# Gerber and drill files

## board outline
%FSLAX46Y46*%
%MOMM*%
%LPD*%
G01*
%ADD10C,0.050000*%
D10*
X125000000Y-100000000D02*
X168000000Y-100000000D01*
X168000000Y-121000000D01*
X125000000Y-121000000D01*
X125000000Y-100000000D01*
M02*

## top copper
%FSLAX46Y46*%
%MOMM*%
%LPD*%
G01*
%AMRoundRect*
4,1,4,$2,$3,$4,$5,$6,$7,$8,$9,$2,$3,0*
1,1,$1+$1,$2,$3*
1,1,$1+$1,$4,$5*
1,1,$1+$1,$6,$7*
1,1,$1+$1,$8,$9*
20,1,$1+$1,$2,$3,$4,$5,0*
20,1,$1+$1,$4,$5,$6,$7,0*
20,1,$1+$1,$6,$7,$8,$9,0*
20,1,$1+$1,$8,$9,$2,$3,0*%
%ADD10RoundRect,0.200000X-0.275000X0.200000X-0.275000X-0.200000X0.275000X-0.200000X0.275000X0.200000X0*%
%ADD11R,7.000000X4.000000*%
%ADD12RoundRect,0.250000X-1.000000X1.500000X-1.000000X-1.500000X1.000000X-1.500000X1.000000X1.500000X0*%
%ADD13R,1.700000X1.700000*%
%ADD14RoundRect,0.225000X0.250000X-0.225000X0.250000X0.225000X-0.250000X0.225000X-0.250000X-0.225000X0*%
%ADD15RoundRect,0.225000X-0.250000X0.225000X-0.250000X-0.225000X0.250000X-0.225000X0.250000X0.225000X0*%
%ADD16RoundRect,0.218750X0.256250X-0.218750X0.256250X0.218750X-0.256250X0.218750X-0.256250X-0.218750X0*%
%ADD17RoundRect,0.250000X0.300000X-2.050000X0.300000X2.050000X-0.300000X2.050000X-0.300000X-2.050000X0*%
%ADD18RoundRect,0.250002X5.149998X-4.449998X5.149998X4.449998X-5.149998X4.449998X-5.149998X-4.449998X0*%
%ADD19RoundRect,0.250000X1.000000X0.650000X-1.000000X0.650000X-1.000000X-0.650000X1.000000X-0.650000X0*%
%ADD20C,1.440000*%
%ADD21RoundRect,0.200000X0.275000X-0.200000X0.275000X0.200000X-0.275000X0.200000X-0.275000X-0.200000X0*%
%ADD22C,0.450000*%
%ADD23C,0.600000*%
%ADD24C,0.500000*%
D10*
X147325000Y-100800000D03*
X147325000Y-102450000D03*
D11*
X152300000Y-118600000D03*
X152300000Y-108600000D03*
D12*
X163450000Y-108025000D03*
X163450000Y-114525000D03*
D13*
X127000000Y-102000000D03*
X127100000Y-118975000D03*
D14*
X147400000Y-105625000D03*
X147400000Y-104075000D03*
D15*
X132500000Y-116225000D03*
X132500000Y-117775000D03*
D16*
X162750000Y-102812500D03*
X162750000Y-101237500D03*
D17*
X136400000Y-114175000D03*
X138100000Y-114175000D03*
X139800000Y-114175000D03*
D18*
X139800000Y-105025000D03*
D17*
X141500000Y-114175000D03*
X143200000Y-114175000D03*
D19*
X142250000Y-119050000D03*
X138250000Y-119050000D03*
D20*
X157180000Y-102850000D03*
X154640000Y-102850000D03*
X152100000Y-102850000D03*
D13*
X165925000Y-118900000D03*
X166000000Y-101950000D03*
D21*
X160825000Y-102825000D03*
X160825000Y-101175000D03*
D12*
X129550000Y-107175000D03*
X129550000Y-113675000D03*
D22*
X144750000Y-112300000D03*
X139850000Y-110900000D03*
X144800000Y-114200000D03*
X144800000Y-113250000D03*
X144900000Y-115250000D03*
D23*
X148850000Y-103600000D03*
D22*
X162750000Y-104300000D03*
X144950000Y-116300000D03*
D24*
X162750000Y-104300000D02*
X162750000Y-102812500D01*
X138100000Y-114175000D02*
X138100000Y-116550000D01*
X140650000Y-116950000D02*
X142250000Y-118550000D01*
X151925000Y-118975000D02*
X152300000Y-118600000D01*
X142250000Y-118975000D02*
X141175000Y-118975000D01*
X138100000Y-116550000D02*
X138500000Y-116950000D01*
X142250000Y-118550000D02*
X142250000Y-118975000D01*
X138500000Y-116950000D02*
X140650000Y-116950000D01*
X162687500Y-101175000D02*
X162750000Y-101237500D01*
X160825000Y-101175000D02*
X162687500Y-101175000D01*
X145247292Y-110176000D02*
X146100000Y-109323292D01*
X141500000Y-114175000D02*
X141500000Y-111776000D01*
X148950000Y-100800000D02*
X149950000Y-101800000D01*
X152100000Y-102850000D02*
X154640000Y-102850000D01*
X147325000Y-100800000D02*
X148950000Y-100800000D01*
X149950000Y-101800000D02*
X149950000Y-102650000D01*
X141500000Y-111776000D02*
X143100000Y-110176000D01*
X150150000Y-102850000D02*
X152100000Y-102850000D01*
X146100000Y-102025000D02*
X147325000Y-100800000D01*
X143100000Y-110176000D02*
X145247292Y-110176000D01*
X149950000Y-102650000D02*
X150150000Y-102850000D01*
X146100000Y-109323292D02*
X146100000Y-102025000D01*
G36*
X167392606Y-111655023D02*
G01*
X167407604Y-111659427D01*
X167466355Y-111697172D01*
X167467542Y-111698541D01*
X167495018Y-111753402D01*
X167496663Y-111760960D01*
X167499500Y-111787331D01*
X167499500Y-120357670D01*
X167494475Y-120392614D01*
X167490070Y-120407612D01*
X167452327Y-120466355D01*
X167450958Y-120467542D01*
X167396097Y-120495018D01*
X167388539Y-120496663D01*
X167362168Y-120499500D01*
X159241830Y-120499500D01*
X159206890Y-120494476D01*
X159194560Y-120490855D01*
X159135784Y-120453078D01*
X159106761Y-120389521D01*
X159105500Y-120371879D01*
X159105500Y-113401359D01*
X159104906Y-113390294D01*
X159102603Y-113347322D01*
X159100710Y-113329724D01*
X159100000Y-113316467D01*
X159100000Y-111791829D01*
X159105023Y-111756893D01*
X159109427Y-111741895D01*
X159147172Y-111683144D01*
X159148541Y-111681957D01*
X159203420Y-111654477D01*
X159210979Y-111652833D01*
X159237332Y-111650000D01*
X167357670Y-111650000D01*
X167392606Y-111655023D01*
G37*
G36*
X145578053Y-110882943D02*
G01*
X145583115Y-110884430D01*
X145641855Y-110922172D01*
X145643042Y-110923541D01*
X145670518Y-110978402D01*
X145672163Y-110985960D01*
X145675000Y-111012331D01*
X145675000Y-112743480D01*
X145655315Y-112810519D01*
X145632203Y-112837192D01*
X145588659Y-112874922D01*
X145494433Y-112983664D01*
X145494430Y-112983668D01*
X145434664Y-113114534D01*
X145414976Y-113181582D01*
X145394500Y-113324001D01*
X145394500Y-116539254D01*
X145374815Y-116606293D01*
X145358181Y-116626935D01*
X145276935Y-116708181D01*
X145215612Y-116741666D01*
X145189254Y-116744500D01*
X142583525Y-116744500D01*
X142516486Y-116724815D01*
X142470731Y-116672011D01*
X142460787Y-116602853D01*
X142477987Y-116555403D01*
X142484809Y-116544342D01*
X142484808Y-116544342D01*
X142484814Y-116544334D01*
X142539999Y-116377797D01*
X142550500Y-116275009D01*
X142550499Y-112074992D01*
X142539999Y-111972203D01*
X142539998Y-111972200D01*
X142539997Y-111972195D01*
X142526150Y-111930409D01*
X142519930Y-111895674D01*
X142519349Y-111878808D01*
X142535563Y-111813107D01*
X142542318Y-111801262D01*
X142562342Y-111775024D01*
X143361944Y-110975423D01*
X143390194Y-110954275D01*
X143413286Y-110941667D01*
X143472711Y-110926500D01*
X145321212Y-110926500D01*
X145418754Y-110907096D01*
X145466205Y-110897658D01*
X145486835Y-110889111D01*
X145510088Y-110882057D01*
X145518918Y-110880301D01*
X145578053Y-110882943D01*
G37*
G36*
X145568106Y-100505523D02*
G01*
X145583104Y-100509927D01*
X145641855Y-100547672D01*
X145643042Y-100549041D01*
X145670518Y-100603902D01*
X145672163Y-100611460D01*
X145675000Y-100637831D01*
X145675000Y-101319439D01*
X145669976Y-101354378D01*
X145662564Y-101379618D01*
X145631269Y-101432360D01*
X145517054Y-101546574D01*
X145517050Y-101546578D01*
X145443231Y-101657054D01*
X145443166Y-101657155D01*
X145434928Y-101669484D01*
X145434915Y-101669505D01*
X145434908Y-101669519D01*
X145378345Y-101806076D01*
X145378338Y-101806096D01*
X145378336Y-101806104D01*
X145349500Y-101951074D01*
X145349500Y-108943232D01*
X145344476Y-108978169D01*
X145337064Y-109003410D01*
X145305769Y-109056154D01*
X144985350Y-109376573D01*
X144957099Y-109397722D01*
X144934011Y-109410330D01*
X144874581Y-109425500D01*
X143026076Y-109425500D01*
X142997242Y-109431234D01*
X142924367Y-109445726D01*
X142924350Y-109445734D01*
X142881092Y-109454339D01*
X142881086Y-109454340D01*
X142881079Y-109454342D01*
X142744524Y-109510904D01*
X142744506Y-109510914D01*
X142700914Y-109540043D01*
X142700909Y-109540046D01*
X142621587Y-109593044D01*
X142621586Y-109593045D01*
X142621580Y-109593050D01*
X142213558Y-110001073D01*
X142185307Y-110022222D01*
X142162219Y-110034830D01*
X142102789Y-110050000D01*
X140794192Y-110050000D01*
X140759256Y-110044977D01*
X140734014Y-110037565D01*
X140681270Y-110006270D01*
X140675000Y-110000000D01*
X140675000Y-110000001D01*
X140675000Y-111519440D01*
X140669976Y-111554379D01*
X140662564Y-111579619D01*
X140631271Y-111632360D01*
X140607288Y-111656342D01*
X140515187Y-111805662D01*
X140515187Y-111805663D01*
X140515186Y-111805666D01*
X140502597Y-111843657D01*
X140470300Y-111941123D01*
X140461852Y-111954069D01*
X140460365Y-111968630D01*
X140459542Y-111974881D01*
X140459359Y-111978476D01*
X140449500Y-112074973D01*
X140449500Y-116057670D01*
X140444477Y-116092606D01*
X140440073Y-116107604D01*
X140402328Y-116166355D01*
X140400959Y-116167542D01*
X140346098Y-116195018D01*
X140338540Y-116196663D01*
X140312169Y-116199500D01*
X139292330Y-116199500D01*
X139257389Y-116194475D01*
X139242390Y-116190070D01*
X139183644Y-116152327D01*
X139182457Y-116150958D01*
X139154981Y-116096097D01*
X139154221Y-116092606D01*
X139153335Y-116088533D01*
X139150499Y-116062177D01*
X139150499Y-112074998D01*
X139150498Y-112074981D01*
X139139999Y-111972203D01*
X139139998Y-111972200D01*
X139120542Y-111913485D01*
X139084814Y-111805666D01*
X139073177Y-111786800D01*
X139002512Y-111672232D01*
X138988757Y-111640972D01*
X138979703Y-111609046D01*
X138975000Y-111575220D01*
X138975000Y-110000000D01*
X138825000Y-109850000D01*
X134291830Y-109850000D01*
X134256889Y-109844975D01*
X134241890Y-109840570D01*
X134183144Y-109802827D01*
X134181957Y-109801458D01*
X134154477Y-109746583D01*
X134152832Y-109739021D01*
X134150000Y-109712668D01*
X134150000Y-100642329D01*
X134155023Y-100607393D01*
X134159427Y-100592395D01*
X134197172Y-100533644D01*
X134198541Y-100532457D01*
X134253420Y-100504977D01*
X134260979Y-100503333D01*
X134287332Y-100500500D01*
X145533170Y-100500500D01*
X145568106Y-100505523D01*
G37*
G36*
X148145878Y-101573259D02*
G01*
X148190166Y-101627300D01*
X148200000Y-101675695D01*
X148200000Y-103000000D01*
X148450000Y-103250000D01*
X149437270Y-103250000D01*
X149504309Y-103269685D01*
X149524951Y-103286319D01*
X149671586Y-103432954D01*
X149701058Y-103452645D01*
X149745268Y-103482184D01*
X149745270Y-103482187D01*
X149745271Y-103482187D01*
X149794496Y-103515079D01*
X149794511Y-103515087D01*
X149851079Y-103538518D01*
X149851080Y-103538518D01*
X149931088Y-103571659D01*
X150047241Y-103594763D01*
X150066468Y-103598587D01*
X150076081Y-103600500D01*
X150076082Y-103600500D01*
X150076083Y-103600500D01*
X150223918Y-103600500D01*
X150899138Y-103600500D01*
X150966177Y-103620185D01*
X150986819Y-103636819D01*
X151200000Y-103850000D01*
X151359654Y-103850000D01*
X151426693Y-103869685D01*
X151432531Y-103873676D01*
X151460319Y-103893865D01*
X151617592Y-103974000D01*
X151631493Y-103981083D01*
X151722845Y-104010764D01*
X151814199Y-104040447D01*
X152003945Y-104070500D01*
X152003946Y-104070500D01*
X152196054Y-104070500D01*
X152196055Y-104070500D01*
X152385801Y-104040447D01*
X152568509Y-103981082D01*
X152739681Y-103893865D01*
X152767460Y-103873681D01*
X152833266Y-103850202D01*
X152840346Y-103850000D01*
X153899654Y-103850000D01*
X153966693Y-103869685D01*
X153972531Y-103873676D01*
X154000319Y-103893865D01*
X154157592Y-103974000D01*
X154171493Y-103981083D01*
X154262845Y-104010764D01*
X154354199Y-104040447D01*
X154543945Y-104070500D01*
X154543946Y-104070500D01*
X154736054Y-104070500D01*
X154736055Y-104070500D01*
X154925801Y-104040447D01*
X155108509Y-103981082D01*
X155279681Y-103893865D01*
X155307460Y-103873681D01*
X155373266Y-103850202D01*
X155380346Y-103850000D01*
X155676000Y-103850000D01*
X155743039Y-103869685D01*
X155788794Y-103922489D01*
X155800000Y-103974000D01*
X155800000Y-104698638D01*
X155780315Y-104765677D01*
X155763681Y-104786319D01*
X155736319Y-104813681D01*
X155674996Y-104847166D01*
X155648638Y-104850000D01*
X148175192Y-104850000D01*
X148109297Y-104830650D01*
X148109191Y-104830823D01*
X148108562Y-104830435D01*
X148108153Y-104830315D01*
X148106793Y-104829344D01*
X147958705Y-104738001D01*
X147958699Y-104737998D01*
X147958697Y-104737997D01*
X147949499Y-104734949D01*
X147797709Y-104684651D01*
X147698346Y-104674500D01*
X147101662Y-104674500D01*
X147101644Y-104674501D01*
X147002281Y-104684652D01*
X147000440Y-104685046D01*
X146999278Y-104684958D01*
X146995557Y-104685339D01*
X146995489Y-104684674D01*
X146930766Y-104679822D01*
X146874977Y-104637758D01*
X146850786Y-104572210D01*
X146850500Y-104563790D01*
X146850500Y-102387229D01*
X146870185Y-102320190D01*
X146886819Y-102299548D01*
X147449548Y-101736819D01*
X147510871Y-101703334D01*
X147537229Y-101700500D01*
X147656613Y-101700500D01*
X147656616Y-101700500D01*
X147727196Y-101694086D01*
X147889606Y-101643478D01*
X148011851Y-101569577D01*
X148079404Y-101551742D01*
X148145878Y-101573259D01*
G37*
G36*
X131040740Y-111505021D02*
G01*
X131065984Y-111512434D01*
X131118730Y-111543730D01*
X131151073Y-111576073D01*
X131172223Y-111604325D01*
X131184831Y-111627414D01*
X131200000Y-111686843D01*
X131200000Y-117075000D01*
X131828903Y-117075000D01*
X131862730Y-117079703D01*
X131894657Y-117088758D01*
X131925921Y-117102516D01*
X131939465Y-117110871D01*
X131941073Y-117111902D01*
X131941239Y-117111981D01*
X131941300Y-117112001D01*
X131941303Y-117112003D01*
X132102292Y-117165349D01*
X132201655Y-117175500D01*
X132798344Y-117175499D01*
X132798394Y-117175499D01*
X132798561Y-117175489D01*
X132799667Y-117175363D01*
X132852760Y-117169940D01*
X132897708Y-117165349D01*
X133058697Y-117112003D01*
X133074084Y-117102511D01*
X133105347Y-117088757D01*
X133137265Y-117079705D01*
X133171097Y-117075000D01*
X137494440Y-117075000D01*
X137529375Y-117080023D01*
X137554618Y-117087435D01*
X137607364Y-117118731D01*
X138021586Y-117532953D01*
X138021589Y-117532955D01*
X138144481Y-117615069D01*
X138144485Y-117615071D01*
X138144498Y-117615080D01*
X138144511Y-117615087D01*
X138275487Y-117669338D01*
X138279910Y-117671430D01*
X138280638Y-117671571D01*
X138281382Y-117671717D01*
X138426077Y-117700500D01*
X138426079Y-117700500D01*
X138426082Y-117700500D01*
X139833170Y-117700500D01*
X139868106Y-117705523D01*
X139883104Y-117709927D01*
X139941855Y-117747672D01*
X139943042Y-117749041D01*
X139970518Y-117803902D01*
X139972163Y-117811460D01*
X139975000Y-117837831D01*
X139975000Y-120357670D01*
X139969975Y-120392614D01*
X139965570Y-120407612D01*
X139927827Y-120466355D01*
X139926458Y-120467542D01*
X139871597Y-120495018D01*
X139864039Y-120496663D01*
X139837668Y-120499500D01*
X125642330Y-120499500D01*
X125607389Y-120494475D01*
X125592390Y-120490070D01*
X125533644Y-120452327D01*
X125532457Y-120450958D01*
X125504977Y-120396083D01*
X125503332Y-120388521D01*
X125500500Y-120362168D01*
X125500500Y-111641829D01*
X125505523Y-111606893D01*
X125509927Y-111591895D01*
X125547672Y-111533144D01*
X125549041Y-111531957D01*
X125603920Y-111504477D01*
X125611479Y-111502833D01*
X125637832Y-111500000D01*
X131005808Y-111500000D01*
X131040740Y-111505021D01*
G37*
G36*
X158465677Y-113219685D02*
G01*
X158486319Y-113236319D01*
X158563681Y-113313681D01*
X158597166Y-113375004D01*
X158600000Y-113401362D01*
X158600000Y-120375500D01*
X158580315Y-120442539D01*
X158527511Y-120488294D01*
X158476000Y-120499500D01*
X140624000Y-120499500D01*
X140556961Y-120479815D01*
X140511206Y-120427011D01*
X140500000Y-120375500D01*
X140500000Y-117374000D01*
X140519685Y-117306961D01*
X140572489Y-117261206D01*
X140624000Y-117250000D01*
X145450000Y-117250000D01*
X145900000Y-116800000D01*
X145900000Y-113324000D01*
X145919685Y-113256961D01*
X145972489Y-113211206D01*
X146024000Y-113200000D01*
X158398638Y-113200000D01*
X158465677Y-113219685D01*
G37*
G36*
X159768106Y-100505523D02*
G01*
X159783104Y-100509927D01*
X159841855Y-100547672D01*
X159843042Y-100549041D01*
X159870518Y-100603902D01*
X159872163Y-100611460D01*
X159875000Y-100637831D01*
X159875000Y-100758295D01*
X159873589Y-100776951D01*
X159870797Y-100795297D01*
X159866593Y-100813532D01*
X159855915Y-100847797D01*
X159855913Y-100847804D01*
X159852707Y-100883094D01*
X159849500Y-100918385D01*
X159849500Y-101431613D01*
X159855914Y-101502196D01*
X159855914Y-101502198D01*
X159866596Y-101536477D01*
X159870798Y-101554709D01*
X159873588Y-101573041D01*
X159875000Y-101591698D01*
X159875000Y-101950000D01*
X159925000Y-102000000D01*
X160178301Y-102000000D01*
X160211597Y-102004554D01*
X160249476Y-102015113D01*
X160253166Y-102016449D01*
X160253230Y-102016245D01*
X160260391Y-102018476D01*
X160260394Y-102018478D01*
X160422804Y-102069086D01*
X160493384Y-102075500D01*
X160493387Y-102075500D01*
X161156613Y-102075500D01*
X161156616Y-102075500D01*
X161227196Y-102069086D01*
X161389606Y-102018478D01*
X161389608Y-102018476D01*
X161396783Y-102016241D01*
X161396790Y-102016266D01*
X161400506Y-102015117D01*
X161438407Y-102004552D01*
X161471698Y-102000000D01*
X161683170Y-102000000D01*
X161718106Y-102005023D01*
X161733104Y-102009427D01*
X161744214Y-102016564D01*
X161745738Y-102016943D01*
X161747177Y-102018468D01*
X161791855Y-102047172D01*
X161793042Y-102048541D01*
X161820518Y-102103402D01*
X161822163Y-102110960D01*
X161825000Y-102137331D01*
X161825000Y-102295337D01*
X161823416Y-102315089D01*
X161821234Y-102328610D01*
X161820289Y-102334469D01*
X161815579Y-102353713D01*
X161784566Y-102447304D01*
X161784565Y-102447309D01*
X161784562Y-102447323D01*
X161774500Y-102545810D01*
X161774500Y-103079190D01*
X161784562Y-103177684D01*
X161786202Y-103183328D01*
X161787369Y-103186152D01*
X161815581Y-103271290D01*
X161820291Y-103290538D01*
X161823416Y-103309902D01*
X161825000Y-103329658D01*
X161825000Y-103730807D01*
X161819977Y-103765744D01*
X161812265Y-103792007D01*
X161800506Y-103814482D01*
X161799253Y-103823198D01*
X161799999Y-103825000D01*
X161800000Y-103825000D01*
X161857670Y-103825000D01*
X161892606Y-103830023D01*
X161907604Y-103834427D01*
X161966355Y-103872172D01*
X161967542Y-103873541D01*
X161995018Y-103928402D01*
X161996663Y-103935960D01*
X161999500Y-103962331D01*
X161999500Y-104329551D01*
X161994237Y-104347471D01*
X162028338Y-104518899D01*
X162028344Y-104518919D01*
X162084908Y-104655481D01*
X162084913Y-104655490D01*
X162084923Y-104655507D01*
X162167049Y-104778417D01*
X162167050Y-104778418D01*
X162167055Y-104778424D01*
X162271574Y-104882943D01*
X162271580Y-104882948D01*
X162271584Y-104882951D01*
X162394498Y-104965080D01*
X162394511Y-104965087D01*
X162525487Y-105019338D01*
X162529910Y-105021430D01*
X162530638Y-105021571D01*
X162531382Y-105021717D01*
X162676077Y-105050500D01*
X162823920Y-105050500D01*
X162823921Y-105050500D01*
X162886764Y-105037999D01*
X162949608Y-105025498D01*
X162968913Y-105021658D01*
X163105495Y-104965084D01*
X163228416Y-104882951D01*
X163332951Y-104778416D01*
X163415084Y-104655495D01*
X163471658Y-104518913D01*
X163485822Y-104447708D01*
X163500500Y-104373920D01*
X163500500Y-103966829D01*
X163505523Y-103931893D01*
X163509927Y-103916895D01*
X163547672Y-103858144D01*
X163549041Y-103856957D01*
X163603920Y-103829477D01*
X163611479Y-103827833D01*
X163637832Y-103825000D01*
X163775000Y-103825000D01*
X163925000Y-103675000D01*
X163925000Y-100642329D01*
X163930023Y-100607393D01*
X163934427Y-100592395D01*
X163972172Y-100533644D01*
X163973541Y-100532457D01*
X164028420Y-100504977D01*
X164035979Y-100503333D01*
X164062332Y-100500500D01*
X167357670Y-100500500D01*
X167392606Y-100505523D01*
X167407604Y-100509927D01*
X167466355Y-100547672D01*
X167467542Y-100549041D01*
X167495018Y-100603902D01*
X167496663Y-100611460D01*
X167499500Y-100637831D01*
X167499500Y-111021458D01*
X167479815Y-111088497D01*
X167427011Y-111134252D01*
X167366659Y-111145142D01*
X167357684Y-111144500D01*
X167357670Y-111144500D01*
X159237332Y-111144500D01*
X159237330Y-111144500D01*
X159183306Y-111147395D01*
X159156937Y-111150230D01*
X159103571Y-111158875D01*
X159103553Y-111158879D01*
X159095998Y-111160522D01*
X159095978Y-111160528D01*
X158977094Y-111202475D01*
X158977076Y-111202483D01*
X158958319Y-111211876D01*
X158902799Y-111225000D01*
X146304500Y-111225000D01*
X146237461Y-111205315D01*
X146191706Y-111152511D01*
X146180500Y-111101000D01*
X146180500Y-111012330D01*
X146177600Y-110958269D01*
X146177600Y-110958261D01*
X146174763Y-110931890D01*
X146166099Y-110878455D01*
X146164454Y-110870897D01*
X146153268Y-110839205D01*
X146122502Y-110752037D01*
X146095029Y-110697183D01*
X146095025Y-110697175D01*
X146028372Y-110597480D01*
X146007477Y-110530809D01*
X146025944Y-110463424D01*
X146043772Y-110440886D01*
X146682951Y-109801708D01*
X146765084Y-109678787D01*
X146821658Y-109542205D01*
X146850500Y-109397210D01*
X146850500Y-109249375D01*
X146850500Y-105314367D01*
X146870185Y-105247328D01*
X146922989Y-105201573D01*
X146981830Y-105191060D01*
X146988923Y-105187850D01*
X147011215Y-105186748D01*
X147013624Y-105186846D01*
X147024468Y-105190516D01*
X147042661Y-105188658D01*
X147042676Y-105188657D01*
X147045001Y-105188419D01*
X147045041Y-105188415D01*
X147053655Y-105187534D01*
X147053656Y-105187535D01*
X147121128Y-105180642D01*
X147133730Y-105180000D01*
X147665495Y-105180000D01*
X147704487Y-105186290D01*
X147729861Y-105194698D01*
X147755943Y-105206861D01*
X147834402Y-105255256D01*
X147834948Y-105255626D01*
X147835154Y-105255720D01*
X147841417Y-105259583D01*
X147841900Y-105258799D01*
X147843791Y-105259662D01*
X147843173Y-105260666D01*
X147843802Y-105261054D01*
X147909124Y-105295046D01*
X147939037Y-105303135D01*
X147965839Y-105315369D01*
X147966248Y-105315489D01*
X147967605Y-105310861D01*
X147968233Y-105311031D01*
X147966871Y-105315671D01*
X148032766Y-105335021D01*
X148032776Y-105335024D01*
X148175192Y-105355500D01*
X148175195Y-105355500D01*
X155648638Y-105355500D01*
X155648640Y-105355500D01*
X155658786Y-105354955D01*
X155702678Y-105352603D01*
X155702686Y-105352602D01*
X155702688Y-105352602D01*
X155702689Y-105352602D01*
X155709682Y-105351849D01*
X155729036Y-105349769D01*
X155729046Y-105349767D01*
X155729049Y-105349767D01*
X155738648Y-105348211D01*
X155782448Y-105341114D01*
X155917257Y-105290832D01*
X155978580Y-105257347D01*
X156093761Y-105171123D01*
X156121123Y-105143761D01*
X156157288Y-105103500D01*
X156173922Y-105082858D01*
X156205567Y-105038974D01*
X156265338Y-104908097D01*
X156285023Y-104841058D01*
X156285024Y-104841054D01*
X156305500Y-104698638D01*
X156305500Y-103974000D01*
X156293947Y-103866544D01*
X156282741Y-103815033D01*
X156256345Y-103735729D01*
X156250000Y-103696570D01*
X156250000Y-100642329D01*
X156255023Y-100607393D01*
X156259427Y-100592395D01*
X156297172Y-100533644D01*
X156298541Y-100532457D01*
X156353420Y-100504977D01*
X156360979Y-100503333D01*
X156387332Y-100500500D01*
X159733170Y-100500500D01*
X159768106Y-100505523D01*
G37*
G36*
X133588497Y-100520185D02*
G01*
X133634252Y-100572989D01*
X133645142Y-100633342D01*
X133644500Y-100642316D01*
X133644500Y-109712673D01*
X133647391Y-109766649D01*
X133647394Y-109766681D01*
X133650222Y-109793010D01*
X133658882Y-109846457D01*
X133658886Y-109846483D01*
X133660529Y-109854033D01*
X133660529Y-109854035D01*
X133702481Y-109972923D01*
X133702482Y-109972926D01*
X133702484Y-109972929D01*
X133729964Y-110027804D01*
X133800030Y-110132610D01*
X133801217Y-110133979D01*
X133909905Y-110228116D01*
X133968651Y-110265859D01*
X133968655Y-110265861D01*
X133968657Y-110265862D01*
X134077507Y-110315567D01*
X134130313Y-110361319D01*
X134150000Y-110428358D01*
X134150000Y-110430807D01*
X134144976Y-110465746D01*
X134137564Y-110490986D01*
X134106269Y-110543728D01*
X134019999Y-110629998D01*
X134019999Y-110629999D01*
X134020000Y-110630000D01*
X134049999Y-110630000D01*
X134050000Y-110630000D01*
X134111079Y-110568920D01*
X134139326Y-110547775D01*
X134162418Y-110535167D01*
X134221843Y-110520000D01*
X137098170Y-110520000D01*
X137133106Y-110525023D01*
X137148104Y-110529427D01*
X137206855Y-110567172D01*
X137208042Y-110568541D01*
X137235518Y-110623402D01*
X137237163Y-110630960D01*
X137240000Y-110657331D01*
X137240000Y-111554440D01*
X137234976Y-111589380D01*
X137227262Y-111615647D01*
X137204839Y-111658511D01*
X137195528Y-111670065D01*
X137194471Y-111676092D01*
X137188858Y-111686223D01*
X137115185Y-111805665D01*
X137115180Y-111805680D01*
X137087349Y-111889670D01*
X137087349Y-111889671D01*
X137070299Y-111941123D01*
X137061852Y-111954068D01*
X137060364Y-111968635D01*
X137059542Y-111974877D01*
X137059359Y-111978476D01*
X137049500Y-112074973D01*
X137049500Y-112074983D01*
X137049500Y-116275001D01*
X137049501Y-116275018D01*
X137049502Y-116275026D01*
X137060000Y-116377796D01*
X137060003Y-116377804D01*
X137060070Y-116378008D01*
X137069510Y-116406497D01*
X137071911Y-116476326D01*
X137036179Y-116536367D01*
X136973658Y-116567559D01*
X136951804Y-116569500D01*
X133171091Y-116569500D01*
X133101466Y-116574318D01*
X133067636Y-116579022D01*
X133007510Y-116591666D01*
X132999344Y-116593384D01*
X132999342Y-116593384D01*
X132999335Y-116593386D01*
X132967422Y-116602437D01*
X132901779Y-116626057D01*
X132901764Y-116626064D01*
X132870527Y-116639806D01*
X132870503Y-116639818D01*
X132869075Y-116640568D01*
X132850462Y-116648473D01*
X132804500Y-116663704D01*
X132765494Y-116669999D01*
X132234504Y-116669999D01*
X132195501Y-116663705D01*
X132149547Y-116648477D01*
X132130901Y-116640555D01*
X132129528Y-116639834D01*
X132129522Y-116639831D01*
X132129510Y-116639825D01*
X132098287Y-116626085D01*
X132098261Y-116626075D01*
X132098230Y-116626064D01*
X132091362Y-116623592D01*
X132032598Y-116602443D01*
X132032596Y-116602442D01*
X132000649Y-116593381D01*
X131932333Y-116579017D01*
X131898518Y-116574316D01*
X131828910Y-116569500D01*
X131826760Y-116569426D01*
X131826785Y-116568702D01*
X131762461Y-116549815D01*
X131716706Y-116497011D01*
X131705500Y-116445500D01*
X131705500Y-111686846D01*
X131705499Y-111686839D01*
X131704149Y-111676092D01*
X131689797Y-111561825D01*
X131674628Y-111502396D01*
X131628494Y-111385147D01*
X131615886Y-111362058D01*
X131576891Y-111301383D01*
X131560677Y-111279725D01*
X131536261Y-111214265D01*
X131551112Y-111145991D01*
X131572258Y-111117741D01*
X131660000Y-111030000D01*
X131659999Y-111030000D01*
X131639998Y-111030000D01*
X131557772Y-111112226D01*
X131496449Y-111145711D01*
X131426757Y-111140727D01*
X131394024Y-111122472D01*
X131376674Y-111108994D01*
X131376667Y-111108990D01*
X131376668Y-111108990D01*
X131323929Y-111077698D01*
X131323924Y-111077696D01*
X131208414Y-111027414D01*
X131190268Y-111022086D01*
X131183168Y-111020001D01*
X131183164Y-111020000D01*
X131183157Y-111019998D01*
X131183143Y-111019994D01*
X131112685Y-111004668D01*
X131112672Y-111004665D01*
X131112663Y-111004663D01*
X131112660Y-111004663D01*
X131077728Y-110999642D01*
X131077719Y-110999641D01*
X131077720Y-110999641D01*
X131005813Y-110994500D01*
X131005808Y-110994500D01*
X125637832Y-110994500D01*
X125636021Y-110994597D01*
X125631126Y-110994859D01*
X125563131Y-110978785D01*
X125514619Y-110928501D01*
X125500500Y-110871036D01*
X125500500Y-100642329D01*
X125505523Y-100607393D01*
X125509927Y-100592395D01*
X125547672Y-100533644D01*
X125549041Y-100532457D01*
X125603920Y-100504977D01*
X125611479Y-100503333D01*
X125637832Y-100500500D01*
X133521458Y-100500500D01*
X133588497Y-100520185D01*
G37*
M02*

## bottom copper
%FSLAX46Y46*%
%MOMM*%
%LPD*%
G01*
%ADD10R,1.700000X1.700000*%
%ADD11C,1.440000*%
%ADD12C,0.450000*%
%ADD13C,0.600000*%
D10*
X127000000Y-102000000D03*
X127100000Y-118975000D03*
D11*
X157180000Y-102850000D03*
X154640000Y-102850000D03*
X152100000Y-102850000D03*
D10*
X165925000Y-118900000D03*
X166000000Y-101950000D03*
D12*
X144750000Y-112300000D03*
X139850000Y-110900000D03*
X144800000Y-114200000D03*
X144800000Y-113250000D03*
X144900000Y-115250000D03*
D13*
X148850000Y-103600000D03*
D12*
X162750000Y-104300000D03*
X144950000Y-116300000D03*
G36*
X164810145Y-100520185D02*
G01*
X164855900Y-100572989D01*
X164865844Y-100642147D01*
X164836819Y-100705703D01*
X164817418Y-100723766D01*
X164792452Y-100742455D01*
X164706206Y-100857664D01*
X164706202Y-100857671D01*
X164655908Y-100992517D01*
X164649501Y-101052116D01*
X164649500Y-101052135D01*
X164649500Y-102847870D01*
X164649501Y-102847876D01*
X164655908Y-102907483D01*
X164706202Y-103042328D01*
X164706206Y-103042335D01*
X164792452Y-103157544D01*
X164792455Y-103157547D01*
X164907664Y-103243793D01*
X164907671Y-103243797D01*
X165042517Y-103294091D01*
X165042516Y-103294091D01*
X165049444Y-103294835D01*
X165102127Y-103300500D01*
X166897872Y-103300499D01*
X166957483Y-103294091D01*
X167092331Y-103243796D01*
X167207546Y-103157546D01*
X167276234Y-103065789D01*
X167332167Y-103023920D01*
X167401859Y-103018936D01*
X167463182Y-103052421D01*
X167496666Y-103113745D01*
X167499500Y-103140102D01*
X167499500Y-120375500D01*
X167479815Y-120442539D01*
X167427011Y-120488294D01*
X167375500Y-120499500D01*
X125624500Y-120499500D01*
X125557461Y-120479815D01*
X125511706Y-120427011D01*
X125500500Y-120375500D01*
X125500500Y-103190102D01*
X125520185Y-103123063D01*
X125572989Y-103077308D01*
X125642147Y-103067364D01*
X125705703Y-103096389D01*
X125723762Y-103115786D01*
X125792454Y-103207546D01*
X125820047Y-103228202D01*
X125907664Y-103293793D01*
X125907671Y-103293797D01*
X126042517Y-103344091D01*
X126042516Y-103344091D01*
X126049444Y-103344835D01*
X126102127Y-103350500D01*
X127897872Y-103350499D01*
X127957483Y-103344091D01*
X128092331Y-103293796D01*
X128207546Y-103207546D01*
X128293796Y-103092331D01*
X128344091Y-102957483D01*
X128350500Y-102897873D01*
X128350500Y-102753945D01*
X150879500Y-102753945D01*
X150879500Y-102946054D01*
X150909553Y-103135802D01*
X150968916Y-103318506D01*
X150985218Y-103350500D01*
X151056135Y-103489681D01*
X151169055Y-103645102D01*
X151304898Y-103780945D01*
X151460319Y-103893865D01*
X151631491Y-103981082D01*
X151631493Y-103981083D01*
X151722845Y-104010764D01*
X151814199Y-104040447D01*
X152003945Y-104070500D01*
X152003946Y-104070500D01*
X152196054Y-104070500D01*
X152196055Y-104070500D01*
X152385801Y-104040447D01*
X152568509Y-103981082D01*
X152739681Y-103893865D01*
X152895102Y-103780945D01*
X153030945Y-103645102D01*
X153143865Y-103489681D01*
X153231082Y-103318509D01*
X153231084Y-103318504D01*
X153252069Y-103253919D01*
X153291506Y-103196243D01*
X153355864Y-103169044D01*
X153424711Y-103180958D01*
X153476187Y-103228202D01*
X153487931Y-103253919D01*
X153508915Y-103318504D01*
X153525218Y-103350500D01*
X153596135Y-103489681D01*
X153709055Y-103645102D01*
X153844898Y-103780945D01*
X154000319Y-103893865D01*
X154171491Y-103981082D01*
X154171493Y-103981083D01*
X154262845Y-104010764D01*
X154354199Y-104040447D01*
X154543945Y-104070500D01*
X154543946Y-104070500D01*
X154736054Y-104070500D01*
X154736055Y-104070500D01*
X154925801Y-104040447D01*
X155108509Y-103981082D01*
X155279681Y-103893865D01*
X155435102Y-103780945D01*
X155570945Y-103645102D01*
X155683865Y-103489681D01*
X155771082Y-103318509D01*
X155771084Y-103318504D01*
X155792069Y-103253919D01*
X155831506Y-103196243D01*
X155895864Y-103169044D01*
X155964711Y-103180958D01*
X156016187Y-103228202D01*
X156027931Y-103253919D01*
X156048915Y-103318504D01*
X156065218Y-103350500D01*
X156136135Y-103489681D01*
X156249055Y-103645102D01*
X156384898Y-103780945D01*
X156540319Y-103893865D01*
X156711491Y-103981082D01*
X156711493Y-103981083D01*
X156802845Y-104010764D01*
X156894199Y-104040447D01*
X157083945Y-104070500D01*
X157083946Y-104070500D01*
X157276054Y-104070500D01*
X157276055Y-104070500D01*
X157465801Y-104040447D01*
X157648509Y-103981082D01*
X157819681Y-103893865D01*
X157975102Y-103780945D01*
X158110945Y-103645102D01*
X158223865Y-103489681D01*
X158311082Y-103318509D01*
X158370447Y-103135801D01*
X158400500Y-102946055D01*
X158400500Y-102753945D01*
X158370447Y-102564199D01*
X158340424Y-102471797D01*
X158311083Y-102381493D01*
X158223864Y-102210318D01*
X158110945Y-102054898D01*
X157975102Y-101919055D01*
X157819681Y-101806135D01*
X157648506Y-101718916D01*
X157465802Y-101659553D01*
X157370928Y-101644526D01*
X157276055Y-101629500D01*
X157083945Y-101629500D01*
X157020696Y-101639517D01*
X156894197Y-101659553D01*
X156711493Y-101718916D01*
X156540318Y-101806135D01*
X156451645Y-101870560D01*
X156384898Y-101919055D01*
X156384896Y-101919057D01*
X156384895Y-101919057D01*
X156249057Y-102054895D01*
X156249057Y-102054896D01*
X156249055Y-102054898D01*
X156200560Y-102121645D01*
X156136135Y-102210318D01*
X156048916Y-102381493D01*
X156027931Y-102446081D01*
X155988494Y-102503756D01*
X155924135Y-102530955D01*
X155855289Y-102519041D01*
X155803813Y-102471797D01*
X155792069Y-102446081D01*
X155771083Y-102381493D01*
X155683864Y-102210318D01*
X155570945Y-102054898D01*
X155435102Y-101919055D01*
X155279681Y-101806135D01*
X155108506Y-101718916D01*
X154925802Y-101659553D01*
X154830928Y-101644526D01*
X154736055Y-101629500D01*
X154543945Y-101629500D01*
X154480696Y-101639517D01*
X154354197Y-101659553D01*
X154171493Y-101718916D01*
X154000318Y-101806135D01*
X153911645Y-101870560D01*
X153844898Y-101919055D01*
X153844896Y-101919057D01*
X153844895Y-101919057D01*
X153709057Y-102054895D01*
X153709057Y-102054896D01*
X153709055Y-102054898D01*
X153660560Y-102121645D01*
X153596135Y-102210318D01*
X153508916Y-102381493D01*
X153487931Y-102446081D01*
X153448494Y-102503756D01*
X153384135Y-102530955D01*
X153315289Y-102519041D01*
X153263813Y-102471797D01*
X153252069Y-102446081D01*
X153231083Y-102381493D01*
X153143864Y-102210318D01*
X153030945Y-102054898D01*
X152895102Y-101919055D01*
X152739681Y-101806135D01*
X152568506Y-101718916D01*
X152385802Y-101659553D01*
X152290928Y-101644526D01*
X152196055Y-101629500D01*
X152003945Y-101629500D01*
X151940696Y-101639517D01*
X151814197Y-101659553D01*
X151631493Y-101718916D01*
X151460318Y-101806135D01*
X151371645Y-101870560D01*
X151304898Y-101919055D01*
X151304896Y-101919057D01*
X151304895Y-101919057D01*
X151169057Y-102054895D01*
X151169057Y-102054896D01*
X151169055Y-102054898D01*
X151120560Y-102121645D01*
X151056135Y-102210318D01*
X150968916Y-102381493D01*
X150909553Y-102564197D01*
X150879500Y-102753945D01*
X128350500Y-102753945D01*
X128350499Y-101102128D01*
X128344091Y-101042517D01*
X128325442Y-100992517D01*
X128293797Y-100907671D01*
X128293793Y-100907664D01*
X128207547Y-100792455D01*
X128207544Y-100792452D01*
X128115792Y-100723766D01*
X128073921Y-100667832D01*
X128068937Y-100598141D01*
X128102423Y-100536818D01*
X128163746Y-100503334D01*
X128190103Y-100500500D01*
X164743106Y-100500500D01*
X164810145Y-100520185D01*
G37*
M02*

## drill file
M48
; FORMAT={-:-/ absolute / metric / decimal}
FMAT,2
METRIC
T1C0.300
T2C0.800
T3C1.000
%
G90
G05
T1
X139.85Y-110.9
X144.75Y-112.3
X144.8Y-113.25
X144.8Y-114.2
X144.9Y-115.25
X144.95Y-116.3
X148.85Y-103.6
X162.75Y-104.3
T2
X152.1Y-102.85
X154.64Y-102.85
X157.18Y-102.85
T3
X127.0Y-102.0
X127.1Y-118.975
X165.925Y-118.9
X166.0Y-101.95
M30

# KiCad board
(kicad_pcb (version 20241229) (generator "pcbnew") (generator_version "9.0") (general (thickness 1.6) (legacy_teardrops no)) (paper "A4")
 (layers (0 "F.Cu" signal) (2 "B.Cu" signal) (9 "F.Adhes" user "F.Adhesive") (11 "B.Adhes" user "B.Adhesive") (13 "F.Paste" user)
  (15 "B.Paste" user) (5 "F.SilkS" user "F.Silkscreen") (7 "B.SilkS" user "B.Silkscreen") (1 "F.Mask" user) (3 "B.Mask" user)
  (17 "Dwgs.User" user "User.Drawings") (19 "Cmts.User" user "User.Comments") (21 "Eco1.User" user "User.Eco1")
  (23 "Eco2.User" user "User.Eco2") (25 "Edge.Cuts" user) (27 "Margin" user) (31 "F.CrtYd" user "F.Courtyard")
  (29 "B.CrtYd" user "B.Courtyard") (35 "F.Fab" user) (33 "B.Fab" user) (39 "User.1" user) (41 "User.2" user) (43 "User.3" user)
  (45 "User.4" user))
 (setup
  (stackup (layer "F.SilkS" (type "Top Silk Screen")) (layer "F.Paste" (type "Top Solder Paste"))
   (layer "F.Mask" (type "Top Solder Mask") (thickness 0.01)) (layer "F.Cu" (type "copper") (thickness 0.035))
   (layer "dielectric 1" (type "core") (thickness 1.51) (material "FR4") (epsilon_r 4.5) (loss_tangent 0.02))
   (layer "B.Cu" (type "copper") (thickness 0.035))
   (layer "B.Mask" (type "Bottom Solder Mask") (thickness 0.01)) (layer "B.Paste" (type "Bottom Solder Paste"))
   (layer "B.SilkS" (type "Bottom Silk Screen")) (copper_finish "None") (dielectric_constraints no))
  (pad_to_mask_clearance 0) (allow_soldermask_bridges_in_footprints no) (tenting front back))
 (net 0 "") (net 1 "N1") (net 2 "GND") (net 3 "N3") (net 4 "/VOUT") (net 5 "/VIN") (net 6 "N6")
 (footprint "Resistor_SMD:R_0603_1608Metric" (layer "F.Cu") (at 147.325 101.625 -90)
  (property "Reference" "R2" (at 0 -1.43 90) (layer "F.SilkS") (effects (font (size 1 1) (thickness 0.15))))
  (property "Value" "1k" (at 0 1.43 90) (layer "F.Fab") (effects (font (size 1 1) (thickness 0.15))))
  (pad "1" smd roundrect (at -0.825 0 270) (size 0.8 0.95) (layers "F.Cu" "F.Mask" "F.Paste") (roundrect_rratio 0.25) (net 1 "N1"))
  (pad "2" smd roundrect (at 0.825 0 270) (size 0.8 0.95) (layers "F.Cu" "F.Mask" "F.Paste") (roundrect_rratio 0.25) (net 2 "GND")))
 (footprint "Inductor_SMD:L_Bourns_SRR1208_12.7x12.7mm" (layer "F.Cu") (at 152.3 113.6 90)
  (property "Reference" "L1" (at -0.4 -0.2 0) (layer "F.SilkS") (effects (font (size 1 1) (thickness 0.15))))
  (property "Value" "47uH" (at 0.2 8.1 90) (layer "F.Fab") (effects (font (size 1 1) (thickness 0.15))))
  (pad "1" smd rect (at -5 0 90) (size 4 7) (layers "F.Cu" "F.Mask" "F.Paste") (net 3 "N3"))
  (pad "2" smd rect (at 5 0 90) (size 4 7) (layers "F.Cu" "F.Mask" "F.Paste") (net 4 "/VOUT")))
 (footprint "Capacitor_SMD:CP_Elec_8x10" (layer "F.Cu") (at 163.45 111.275 -90)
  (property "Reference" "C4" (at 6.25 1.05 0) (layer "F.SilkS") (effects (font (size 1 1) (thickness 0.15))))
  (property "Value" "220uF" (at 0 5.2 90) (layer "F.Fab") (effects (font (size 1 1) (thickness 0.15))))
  (pad "1" smd roundrect (at -3.25 0 270) (size 3.5 2.5) (layers "F.Cu" "F.Mask" "F.Paste") (roundrect_rratio 0.1) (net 4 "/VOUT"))
  (pad "2" smd roundrect (at 3.25 0 270) (size 3.5 2.5) (layers "F.Cu" "F.Mask" "F.Paste") (roundrect_rratio 0.1) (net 2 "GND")))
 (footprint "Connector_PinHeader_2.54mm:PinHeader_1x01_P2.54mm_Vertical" (layer "F.Cu") (at 127 102)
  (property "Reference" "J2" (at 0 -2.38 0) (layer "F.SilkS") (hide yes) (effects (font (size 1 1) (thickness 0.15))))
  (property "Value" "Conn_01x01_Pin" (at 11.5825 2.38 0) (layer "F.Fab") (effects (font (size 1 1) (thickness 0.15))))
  (pad "1" thru_hole rect (at 0 0) (size 1.7 1.7) (drill 1) (layers "*.Cu" "*.Mask") (remove_unused_layers no) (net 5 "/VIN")))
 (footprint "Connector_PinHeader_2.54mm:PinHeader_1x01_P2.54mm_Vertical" (layer "F.Cu") (at 127.1 118.975)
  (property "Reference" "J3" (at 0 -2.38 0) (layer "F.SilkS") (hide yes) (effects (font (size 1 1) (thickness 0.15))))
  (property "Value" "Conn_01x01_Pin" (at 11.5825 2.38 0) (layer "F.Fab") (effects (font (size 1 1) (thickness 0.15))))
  (pad "1" thru_hole rect (at 0 0) (size 1.7 1.7) (drill 1) (layers "*.Cu" "*.Mask") (remove_unused_layers no) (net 2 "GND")))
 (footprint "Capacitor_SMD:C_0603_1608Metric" (layer "F.Cu") (at 147.4 104.85 90)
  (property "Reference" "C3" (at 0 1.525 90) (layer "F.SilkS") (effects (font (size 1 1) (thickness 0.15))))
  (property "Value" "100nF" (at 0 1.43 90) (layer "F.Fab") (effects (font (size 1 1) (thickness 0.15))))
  (pad "1" smd roundrect (at -0.775 0 90) (size 0.9 0.95) (layers "F.Cu" "F.Mask" "F.Paste") (roundrect_rratio 0.25) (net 4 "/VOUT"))
  (pad "2" smd roundrect (at 0.775 0 90) (size 0.9 0.95) (layers "F.Cu" "F.Mask" "F.Paste") (roundrect_rratio 0.25) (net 2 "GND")))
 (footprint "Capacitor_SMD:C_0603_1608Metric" (layer "F.Cu") (at 132.5 117 -90)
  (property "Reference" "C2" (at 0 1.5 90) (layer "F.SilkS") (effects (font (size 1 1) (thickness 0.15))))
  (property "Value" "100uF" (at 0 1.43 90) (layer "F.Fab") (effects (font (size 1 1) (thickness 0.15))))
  (pad "1" smd roundrect (at -0.775 0 270) (size 0.9 0.95) (layers "F.Cu" "F.Mask" "F.Paste") (roundrect_rratio 0.25) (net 5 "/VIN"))
  (pad "2" smd roundrect (at 0.775 0 270) (size 0.9 0.95) (layers "F.Cu" "F.Mask" "F.Paste") (roundrect_rratio 0.25) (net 2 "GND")))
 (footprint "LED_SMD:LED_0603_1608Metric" (layer "F.Cu") (at 162.75 102.025 90)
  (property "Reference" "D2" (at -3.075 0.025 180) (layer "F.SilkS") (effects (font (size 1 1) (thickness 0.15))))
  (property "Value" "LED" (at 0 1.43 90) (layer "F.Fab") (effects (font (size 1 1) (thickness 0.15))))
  (pad "1" smd roundrect (at -0.7875 0 90) (size 0.875 0.95) (layers "F.Cu" "F.Mask" "F.Paste") (roundrect_rratio 0.25) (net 2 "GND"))
  (pad "2" smd roundrect (at 0.7875 0 90) (size 0.875 0.95) (layers "F.Cu" "F.Mask" "F.Paste") (roundrect_rratio 0.25) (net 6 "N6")))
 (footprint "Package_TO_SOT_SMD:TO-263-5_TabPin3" (layer "F.Cu") (at 139.8 106.525 90)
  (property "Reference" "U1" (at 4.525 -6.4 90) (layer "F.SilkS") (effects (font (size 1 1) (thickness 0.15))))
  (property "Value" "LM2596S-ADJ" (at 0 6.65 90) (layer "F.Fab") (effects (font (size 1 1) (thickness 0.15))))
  (pad "" smd roundrect (at -0.925 -2.775 90) (size 4.55 5.25) (layers "F.Paste") (roundrect_rratio 0.054945))
  (pad "" smd roundrect (at -0.925 2.775 90) (size 4.55 5.25) (layers "F.Paste") (roundrect_rratio 0.054945))
  (pad "" smd roundrect (at 3.925 -2.775 90) (size 4.55 5.25) (layers "F.Paste") (roundrect_rratio 0.054945))
  (pad "" smd roundrect (at 3.925 2.775 90) (size 4.55 5.25) (layers "F.Paste") (roundrect_rratio 0.054945))
  (pad "1" smd roundrect (at -7.65 -3.4 90) (size 4.6 1.1) (layers "F.Cu" "F.Mask" "F.Paste") (roundrect_rratio 0.227273) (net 5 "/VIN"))
  (pad "2" smd roundrect (at -7.65 -1.7 90) (size 4.6 1.1) (layers "F.Cu" "F.Mask" "F.Paste") (roundrect_rratio 0.227273) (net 3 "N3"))
  (pad "3" smd roundrect (at -7.65 0 90) (size 4.6 1.1) (layers "F.Cu" "F.Mask" "F.Paste") (roundrect_rratio 0.227273) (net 2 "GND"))
  (pad "3" smd roundrect (at 1.5 0 90) (size 9.4 10.8) (layers "F.Cu" "F.Mask") (roundrect_rratio 0.026596) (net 2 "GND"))
  (pad "4" smd roundrect (at -7.65 1.7 90) (size 4.6 1.1) (layers "F.Cu" "F.Mask" "F.Paste") (roundrect_rratio 0.227273) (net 1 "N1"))
  (pad "5" smd roundrect (at -7.65 3.4 90) (size 4.6 1.1) (layers "F.Cu" "F.Mask" "F.Paste") (roundrect_rratio 0.227273) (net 2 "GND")))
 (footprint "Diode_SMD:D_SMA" (layer "F.Cu") (at 140.25 119.05 180)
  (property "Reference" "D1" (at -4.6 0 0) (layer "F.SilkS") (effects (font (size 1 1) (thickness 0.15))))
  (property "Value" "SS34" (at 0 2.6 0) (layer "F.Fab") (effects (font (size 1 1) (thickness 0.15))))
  (pad "1" smd roundrect (at -2 0 180) (size 2.5 1.8) (layers "F.Cu" "F.Mask" "F.Paste") (roundrect_rratio 0.1388888889) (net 3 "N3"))
  (pad "2" smd roundrect (at 2 0 180) (size 2.5 1.8) (layers "F.Cu" "F.Mask" "F.Paste") (roundrect_rratio 0.1388888889) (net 2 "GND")))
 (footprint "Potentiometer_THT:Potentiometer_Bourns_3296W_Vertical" (layer "F.Cu") (at 157.18 102.85)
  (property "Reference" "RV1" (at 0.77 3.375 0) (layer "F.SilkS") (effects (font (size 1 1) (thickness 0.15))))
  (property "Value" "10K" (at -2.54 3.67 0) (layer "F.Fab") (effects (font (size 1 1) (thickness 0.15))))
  (pad "1" thru_hole circle (at 0 0) (size 1.44 1.44) (drill 0.8) (layers "*.Cu" "*.Mask") (remove_unused_layers no) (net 4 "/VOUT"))
  (pad "2" thru_hole circle (at -2.54 0) (size 1.44 1.44) (drill 0.8) (layers "*.Cu" "*.Mask") (remove_unused_layers no) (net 1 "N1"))
  (pad "3" thru_hole circle (at -5.08 0) (size 1.44 1.44) (drill 0.8) (layers "*.Cu" "*.Mask") (remove_unused_layers no) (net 1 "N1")))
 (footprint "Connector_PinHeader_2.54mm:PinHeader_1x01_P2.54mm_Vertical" (layer "F.Cu") (at 165.925 118.9)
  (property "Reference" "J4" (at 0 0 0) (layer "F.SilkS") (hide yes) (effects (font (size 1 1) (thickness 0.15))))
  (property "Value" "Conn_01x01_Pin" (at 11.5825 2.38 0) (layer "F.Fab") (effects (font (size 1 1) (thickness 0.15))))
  (pad "1" thru_hole rect (at 0 0) (size 1.7 1.7) (drill 1) (layers "*.Cu" "*.Mask") (remove_unused_layers no) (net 2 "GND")))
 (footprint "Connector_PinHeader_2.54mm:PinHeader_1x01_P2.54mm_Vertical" (layer "F.Cu") (at 166 101.95)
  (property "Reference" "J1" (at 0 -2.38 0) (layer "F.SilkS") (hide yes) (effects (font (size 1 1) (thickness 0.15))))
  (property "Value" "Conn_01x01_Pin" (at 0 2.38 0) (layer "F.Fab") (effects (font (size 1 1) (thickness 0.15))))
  (pad "1" thru_hole rect (at 0 0) (size 1.7 1.7) (drill 1) (layers "*.Cu" "*.Mask") (remove_unused_layers no) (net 4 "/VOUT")))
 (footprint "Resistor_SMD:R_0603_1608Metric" (layer "F.Cu") (at 160.825 102 90)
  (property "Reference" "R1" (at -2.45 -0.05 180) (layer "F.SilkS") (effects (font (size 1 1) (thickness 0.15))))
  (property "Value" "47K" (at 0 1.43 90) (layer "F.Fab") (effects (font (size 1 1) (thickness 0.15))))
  (pad "1" smd roundrect (at -0.825 0 90) (size 0.8 0.95) (layers "F.Cu" "F.Mask" "F.Paste") (roundrect_rratio 0.25) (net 4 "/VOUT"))
  (pad "2" smd roundrect (at 0.825 0 90) (size 0.8 0.95) (layers "F.Cu" "F.Mask" "F.Paste") (roundrect_rratio 0.25) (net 6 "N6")))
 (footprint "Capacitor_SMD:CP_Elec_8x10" (layer "F.Cu") (at 129.55 110.425 -90)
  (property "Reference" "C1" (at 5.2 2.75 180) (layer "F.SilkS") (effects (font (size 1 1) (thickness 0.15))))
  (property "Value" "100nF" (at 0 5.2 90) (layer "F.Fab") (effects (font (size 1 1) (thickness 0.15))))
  (pad "1" smd roundrect (at -3.25 0 270) (size 3.5 2.5) (layers "F.Cu" "F.Mask" "F.Paste") (roundrect_rratio 0.1) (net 5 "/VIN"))
  (pad "2" smd roundrect (at 3.25 0 270) (size 3.5 2.5) (layers "F.Cu" "F.Mask" "F.Paste") (roundrect_rratio 0.1) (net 2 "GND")))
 (gr_rect (start 125 100) (end 168 121) (stroke (width 0.05) (type default)) (fill no) (layer "Edge.Cuts"))
 (segment (start 162.75 104.3) (end 162.75 102.8125) (width 0.5) (layer "F.Cu") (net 2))
 (via (at 144.75 112.3) (size 0.45) (drill 0.3) (layers "F.Cu" "B.Cu") (free yes) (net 2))
 (via (at 139.85 110.9) (size 0.45) (drill 0.3) (layers "F.Cu" "B.Cu") (free yes) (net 2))
 (via (at 144.8 114.2) (size 0.45) (drill 0.3) (layers "F.Cu" "B.Cu") (free yes) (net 2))
 (via (at 144.8 113.25) (size 0.45) (drill 0.3) (layers "F.Cu" "B.Cu") (free yes) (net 2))
 (via (at 144.9 115.25) (size 0.45) (drill 0.3) (layers "F.Cu" "B.Cu") (free yes) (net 2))
 (via (at 148.85 103.6) (size 0.6) (drill 0.3) (layers "F.Cu" "B.Cu") (free yes) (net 2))
 (via (at 162.75 104.3) (size 0.45) (drill 0.3) (layers "F.Cu" "B.Cu") (free yes) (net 2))
 (via (at 144.95 116.3) (size 0.45) (drill 0.3) (layers "F.Cu" "B.Cu") (free yes) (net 2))
 (segment (start 138.1 114.175) (end 138.1 116.55) (width 0.5) (layer "F.Cu") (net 3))
 (segment (start 140.65 116.95) (end 142.25 118.55) (width 0.5) (layer "F.Cu") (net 3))
 (segment (start 151.925 118.975) (end 152.3 118.6) (width 0.5) (layer "F.Cu") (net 3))
 (segment (start 142.25 118.975) (end 141.175 118.975) (width 0.5) (layer "F.Cu") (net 3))
 (segment (start 138.1 116.55) (end 138.5 116.95) (width 0.5) (layer "F.Cu") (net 3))
 (segment (start 142.25 118.55) (end 142.25 118.975) (width 0.5) (layer "F.Cu") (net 3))
 (segment (start 138.5 116.95) (end 140.65 116.95) (width 0.5) (layer "F.Cu") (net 3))
 (segment (start 162.6875 101.175) (end 162.75 101.2375) (width 0.5) (layer "F.Cu") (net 6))
 (segment (start 160.825 101.175) (end 162.6875 101.175) (width 0.5) (layer "F.Cu") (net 6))
 (segment (start 145.247292 110.176) (end 146.1 109.323292) (width 0.5) (layer "F.Cu") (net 1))
 (segment (start 141.5 114.175) (end 141.5 111.776) (width 0.5) (layer "F.Cu") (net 1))
 (segment (start 148.95 100.8) (end 149.95 101.8) (width 0.5) (layer "F.Cu") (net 1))
 (segment (start 152.1 102.85) (end 154.64 102.85) (width 0.5) (layer "F.Cu") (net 1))
 (segment (start 147.325 100.8) (end 148.95 100.8) (width 0.5) (layer "F.Cu") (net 1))
 (segment (start 149.95 101.8) (end 149.95 102.65) (width 0.5) (layer "F.Cu") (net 1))
 (segment (start 141.5 111.776) (end 143.1 110.176) (width 0.5) (layer "F.Cu") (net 1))
 (segment (start 150.15 102.85) (end 152.1 102.85) (width 0.5) (layer "F.Cu") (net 1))
 (segment (start 146.1 102.025) (end 147.325 100.8) (width 0.5) (layer "F.Cu") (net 1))
 (segment (start 143.1 110.176) (end 145.247292 110.176) (width 0.5) (layer "F.Cu") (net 1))
 (segment (start 149.95 102.65) (end 150.15 102.85) (width 0.5) (layer "F.Cu") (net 1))
 (segment (start 146.1 109.323292) (end 146.1 102.025) (width 0.5) (layer "F.Cu") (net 1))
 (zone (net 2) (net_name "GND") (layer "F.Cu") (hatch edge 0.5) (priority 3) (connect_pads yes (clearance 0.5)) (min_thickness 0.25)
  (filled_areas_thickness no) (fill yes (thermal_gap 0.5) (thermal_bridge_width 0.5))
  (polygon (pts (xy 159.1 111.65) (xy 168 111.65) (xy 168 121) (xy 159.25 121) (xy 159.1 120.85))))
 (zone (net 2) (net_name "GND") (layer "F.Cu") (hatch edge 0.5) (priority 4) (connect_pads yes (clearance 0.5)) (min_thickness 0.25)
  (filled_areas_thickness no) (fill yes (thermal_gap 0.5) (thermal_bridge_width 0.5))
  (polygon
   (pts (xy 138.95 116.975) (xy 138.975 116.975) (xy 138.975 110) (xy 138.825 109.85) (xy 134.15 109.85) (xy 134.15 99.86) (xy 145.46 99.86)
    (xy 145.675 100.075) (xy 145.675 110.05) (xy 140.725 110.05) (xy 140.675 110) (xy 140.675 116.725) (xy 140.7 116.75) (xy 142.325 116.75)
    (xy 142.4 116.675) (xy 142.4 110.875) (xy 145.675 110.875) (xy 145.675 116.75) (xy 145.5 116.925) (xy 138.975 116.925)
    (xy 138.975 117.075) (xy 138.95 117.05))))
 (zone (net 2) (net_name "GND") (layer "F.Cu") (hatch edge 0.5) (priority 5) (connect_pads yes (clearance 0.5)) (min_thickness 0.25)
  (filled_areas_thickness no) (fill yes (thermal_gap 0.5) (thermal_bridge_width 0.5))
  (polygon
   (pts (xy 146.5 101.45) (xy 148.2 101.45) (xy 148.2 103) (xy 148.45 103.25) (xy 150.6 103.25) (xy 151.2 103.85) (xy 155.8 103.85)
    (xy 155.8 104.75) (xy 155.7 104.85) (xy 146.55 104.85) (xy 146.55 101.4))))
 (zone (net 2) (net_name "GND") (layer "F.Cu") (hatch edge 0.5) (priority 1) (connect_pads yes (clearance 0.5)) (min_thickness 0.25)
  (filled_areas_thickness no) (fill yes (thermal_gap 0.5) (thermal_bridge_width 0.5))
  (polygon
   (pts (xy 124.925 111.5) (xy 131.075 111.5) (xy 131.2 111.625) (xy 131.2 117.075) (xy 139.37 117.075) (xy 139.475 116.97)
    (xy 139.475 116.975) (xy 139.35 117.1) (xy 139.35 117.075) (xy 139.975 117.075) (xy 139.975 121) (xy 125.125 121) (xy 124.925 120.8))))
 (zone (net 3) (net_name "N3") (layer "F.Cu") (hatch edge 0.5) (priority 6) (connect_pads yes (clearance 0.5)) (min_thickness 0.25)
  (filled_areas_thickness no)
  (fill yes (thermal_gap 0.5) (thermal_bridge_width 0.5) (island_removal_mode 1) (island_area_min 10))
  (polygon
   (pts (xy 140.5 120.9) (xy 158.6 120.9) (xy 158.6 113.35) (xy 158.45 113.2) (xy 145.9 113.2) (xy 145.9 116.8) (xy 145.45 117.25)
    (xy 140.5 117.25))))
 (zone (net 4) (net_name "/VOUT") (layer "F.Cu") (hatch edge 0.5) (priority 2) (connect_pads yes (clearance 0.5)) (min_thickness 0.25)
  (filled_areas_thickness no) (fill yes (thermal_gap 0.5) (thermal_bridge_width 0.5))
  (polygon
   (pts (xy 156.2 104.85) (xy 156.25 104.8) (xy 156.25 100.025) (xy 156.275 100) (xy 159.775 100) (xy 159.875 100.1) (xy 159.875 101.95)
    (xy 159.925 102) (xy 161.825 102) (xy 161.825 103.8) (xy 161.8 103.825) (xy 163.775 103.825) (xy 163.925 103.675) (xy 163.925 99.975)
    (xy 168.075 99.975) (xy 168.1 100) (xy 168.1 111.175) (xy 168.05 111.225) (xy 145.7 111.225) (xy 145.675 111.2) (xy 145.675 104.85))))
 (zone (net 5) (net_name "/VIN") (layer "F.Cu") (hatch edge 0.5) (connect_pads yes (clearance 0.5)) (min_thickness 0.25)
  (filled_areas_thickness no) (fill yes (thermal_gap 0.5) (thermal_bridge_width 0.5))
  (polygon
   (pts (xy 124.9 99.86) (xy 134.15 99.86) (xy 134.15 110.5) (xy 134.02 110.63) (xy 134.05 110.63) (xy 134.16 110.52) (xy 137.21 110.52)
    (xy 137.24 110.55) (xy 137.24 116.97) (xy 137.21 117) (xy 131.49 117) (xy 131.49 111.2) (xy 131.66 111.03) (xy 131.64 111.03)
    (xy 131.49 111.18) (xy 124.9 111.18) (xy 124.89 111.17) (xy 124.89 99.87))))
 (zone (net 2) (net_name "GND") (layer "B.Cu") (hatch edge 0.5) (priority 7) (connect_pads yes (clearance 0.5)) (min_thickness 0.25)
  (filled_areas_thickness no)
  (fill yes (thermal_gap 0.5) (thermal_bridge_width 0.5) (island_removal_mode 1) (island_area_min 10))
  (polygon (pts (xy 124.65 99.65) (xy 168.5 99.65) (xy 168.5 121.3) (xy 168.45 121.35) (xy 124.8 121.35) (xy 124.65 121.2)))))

